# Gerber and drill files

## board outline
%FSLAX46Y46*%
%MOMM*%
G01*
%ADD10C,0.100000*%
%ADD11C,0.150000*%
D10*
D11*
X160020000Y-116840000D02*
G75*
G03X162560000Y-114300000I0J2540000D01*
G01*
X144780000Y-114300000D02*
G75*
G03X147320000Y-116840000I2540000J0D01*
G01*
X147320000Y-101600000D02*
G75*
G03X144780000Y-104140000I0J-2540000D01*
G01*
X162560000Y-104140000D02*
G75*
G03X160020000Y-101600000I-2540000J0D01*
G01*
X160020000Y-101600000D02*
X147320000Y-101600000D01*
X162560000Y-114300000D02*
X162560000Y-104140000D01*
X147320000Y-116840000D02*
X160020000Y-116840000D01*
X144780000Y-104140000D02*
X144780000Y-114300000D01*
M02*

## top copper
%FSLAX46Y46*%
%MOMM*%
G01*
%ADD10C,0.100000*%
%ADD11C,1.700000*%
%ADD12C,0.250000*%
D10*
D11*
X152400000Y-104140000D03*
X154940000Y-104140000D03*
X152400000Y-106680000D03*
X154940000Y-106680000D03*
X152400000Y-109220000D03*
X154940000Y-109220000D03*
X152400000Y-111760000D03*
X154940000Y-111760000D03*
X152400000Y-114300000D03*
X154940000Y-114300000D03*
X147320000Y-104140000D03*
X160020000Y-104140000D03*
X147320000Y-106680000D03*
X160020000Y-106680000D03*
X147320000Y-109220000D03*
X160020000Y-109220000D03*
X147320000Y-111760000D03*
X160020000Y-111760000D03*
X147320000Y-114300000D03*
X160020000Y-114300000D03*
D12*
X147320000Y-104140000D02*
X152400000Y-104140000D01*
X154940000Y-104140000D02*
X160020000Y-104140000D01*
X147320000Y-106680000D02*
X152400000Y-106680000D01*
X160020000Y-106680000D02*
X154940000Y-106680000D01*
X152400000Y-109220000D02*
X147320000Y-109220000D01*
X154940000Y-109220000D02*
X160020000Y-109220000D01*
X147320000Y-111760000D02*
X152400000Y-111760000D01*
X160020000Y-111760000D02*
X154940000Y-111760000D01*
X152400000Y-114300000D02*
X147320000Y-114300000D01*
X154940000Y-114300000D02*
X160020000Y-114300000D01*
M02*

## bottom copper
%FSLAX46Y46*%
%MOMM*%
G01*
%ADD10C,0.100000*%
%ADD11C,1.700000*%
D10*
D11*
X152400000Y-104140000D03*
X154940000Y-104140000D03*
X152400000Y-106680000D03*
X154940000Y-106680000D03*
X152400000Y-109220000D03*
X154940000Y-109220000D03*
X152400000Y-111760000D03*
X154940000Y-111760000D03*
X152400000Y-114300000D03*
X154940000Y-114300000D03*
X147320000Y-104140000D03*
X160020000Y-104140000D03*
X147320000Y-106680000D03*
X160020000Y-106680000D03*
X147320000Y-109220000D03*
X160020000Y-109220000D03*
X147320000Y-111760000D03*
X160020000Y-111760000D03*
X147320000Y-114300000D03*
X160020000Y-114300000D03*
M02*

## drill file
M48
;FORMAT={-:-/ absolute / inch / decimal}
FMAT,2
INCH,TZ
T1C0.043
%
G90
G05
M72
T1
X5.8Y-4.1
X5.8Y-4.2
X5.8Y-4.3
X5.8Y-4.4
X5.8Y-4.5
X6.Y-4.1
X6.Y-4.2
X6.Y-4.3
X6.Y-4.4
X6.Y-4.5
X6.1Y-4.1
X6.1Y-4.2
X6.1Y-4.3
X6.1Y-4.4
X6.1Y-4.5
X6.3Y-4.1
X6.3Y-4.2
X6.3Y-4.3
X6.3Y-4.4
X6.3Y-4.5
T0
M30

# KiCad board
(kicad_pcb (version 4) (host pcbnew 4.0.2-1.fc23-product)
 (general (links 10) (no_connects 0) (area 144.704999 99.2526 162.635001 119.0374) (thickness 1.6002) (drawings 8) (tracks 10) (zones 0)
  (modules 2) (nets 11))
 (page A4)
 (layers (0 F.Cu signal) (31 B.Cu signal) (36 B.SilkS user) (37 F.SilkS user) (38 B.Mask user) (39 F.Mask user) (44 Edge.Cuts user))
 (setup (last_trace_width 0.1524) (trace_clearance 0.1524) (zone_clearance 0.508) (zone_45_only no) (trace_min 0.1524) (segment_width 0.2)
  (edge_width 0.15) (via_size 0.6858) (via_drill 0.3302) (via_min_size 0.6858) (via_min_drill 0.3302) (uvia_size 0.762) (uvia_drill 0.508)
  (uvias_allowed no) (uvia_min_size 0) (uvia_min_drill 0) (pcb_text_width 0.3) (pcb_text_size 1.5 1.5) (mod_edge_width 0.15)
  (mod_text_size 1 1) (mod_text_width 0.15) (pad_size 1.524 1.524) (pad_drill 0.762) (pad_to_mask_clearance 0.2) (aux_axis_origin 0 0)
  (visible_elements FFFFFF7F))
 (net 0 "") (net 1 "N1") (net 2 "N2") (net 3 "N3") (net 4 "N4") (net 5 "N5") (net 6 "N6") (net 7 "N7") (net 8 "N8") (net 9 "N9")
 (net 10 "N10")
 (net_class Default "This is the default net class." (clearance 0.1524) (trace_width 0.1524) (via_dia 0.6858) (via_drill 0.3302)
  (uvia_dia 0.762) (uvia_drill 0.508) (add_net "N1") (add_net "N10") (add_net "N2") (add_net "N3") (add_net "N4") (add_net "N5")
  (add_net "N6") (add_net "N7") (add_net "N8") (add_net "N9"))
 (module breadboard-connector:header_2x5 (layer F.Cu) (at 152.4 104.14)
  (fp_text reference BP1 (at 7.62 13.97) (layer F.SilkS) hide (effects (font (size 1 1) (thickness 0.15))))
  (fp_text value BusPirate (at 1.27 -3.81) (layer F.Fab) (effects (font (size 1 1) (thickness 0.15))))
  (pad 1 thru_hole circle (at 0 0) (size 1.7 1.7) (drill 1.1) (layers *.Cu *.Mask F.SilkS) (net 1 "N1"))
  (pad 2 thru_hole circle (at 2.54 0) (size 1.7 1.7) (drill 1.1) (layers *.Cu *.Mask F.SilkS) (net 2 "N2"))
  (pad 3 thru_hole circle (at 0 2.54) (size 1.7 1.7) (drill 1.1) (layers *.Cu *.Mask F.SilkS) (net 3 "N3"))
  (pad 4 thru_hole circle (at 2.54 2.54) (size 1.7 1.7) (drill 1.1) (layers *.Cu *.Mask F.SilkS) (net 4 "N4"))
  (pad 5 thru_hole circle (at 0 5.08) (size 1.7 1.7) (drill 1.1) (layers *.Cu *.Mask F.SilkS) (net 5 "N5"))
  (pad 6 thru_hole circle (at 2.54 5.08) (size 1.7 1.7) (drill 1.1) (layers *.Cu *.Mask F.SilkS) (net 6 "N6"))
  (pad 7 thru_hole circle (at 0 7.62) (size 1.7 1.7) (drill 1.1) (layers *.Cu *.Mask F.SilkS) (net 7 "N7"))
  (pad 8 thru_hole circle (at 2.54 7.62) (size 1.7 1.7) (drill 1.1) (layers *.Cu *.Mask F.SilkS) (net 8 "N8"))
  (pad 9 thru_hole circle (at 0 10.16) (size 1.7 1.7) (drill 1.1) (layers *.Cu *.Mask F.SilkS) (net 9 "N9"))
  (pad 10 thru_hole circle (at 2.54 10.16) (size 1.7 1.7) (drill 1.1) (layers *.Cu *.Mask F.SilkS) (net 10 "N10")))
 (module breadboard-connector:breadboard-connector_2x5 (layer F.Cu) (at 147.32 104.14)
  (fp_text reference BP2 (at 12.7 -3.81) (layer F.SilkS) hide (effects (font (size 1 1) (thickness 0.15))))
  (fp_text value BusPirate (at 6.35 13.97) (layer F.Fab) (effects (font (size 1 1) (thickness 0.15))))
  (pad 1 thru_hole circle (at 0 0) (size 1.7 1.7) (drill 1.1) (layers *.Cu *.Mask F.SilkS) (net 1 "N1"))
  (pad 2 thru_hole circle (at 12.7 0) (size 1.7 1.7) (drill 1.1) (layers *.Cu *.Mask F.SilkS) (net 2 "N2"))
  (pad 3 thru_hole circle (at 0 2.54) (size 1.7 1.7) (drill 1.1) (layers *.Cu *.Mask F.SilkS) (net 3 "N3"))
  (pad 4 thru_hole circle (at 12.7 2.54) (size 1.7 1.7) (drill 1.1) (layers *.Cu *.Mask F.SilkS) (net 4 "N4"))
  (pad 5 thru_hole circle (at 0 5.08) (size 1.7 1.7) (drill 1.1) (layers *.Cu *.Mask F.SilkS) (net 5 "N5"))
  (pad 6 thru_hole circle (at 12.7 5.08) (size 1.7 1.7) (drill 1.1) (layers *.Cu *.Mask F.SilkS) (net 6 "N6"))
  (pad 7 thru_hole circle (at 0 7.62) (size 1.7 1.7) (drill 1.1) (layers *.Cu *.Mask F.SilkS) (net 7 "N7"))
  (pad 8 thru_hole circle (at 12.7 7.62) (size 1.7 1.7) (drill 1.1) (layers *.Cu *.Mask F.SilkS) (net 8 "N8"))
  (pad 9 thru_hole circle (at 0 10.16) (size 1.7 1.7) (drill 1.1) (layers *.Cu *.Mask F.SilkS) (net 9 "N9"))
  (pad 10 thru_hole circle (at 12.7 10.16) (size 1.7 1.7) (drill 1.1) (layers *.Cu *.Mask F.SilkS) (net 10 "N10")))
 (gr_arc (start 160.02 114.3) (end 162.56 114.3) (angle 90) (layer Edge.Cuts) (width 0.15))
 (gr_arc (start 147.32 114.3) (end 147.32 116.84) (angle 90) (layer Edge.Cuts) (width 0.15))
 (gr_arc (start 147.32 104.14) (end 144.78 104.14) (angle 90) (layer Edge.Cuts) (width 0.15))
 (gr_arc (start 160.02 104.14) (end 160.02 101.6) (angle 90) (layer Edge.Cuts) (width 0.15))
 (gr_line (start 160.02 101.6) (end 147.32 101.6) (angle 90) (layer Edge.Cuts) (width 0.15))
 (gr_line (start 162.56 114.3) (end 162.56 104.14) (angle 90) (layer Edge.Cuts) (width 0.15))
 (gr_line (start 147.32 116.84) (end 160.02 116.84) (angle 90) (layer Edge.Cuts) (width 0.15))
 (gr_line (start 144.78 104.14) (end 144.78 114.3) (angle 90) (layer Edge.Cuts) (width 0.15))
 (segment (start 147.32 104.14) (end 152.4 104.14) (width 0.25) (layer F.Cu) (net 1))
 (segment (start 154.94 104.14) (end 160.02 104.14) (width 0.25) (layer F.Cu) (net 2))
 (segment (start 147.32 106.68) (end 152.4 106.68) (width 0.25) (layer F.Cu) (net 3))
 (segment (start 160.02 106.68) (end 154.94 106.68) (width 0.25) (layer F.Cu) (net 4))
 (segment (start 152.4 109.22) (end 147.32 109.22) (width 0.25) (layer F.Cu) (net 5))
 (segment (start 154.94 109.22) (end 160.02 109.22) (width 0.25) (layer F.Cu) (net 6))
 (segment (start 147.32 111.76) (end 152.4 111.76) (width 0.25) (layer F.Cu) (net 7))
 (segment (start 160.02 111.76) (end 154.94 111.76) (width 0.25) (layer F.Cu) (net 8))
 (segment (start 152.4 114.3) (end 147.32 114.3) (width 0.25) (layer F.Cu) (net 9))
 (segment (start 154.94 114.3) (end 160.02 114.3) (width 0.25) (layer F.Cu) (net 10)))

